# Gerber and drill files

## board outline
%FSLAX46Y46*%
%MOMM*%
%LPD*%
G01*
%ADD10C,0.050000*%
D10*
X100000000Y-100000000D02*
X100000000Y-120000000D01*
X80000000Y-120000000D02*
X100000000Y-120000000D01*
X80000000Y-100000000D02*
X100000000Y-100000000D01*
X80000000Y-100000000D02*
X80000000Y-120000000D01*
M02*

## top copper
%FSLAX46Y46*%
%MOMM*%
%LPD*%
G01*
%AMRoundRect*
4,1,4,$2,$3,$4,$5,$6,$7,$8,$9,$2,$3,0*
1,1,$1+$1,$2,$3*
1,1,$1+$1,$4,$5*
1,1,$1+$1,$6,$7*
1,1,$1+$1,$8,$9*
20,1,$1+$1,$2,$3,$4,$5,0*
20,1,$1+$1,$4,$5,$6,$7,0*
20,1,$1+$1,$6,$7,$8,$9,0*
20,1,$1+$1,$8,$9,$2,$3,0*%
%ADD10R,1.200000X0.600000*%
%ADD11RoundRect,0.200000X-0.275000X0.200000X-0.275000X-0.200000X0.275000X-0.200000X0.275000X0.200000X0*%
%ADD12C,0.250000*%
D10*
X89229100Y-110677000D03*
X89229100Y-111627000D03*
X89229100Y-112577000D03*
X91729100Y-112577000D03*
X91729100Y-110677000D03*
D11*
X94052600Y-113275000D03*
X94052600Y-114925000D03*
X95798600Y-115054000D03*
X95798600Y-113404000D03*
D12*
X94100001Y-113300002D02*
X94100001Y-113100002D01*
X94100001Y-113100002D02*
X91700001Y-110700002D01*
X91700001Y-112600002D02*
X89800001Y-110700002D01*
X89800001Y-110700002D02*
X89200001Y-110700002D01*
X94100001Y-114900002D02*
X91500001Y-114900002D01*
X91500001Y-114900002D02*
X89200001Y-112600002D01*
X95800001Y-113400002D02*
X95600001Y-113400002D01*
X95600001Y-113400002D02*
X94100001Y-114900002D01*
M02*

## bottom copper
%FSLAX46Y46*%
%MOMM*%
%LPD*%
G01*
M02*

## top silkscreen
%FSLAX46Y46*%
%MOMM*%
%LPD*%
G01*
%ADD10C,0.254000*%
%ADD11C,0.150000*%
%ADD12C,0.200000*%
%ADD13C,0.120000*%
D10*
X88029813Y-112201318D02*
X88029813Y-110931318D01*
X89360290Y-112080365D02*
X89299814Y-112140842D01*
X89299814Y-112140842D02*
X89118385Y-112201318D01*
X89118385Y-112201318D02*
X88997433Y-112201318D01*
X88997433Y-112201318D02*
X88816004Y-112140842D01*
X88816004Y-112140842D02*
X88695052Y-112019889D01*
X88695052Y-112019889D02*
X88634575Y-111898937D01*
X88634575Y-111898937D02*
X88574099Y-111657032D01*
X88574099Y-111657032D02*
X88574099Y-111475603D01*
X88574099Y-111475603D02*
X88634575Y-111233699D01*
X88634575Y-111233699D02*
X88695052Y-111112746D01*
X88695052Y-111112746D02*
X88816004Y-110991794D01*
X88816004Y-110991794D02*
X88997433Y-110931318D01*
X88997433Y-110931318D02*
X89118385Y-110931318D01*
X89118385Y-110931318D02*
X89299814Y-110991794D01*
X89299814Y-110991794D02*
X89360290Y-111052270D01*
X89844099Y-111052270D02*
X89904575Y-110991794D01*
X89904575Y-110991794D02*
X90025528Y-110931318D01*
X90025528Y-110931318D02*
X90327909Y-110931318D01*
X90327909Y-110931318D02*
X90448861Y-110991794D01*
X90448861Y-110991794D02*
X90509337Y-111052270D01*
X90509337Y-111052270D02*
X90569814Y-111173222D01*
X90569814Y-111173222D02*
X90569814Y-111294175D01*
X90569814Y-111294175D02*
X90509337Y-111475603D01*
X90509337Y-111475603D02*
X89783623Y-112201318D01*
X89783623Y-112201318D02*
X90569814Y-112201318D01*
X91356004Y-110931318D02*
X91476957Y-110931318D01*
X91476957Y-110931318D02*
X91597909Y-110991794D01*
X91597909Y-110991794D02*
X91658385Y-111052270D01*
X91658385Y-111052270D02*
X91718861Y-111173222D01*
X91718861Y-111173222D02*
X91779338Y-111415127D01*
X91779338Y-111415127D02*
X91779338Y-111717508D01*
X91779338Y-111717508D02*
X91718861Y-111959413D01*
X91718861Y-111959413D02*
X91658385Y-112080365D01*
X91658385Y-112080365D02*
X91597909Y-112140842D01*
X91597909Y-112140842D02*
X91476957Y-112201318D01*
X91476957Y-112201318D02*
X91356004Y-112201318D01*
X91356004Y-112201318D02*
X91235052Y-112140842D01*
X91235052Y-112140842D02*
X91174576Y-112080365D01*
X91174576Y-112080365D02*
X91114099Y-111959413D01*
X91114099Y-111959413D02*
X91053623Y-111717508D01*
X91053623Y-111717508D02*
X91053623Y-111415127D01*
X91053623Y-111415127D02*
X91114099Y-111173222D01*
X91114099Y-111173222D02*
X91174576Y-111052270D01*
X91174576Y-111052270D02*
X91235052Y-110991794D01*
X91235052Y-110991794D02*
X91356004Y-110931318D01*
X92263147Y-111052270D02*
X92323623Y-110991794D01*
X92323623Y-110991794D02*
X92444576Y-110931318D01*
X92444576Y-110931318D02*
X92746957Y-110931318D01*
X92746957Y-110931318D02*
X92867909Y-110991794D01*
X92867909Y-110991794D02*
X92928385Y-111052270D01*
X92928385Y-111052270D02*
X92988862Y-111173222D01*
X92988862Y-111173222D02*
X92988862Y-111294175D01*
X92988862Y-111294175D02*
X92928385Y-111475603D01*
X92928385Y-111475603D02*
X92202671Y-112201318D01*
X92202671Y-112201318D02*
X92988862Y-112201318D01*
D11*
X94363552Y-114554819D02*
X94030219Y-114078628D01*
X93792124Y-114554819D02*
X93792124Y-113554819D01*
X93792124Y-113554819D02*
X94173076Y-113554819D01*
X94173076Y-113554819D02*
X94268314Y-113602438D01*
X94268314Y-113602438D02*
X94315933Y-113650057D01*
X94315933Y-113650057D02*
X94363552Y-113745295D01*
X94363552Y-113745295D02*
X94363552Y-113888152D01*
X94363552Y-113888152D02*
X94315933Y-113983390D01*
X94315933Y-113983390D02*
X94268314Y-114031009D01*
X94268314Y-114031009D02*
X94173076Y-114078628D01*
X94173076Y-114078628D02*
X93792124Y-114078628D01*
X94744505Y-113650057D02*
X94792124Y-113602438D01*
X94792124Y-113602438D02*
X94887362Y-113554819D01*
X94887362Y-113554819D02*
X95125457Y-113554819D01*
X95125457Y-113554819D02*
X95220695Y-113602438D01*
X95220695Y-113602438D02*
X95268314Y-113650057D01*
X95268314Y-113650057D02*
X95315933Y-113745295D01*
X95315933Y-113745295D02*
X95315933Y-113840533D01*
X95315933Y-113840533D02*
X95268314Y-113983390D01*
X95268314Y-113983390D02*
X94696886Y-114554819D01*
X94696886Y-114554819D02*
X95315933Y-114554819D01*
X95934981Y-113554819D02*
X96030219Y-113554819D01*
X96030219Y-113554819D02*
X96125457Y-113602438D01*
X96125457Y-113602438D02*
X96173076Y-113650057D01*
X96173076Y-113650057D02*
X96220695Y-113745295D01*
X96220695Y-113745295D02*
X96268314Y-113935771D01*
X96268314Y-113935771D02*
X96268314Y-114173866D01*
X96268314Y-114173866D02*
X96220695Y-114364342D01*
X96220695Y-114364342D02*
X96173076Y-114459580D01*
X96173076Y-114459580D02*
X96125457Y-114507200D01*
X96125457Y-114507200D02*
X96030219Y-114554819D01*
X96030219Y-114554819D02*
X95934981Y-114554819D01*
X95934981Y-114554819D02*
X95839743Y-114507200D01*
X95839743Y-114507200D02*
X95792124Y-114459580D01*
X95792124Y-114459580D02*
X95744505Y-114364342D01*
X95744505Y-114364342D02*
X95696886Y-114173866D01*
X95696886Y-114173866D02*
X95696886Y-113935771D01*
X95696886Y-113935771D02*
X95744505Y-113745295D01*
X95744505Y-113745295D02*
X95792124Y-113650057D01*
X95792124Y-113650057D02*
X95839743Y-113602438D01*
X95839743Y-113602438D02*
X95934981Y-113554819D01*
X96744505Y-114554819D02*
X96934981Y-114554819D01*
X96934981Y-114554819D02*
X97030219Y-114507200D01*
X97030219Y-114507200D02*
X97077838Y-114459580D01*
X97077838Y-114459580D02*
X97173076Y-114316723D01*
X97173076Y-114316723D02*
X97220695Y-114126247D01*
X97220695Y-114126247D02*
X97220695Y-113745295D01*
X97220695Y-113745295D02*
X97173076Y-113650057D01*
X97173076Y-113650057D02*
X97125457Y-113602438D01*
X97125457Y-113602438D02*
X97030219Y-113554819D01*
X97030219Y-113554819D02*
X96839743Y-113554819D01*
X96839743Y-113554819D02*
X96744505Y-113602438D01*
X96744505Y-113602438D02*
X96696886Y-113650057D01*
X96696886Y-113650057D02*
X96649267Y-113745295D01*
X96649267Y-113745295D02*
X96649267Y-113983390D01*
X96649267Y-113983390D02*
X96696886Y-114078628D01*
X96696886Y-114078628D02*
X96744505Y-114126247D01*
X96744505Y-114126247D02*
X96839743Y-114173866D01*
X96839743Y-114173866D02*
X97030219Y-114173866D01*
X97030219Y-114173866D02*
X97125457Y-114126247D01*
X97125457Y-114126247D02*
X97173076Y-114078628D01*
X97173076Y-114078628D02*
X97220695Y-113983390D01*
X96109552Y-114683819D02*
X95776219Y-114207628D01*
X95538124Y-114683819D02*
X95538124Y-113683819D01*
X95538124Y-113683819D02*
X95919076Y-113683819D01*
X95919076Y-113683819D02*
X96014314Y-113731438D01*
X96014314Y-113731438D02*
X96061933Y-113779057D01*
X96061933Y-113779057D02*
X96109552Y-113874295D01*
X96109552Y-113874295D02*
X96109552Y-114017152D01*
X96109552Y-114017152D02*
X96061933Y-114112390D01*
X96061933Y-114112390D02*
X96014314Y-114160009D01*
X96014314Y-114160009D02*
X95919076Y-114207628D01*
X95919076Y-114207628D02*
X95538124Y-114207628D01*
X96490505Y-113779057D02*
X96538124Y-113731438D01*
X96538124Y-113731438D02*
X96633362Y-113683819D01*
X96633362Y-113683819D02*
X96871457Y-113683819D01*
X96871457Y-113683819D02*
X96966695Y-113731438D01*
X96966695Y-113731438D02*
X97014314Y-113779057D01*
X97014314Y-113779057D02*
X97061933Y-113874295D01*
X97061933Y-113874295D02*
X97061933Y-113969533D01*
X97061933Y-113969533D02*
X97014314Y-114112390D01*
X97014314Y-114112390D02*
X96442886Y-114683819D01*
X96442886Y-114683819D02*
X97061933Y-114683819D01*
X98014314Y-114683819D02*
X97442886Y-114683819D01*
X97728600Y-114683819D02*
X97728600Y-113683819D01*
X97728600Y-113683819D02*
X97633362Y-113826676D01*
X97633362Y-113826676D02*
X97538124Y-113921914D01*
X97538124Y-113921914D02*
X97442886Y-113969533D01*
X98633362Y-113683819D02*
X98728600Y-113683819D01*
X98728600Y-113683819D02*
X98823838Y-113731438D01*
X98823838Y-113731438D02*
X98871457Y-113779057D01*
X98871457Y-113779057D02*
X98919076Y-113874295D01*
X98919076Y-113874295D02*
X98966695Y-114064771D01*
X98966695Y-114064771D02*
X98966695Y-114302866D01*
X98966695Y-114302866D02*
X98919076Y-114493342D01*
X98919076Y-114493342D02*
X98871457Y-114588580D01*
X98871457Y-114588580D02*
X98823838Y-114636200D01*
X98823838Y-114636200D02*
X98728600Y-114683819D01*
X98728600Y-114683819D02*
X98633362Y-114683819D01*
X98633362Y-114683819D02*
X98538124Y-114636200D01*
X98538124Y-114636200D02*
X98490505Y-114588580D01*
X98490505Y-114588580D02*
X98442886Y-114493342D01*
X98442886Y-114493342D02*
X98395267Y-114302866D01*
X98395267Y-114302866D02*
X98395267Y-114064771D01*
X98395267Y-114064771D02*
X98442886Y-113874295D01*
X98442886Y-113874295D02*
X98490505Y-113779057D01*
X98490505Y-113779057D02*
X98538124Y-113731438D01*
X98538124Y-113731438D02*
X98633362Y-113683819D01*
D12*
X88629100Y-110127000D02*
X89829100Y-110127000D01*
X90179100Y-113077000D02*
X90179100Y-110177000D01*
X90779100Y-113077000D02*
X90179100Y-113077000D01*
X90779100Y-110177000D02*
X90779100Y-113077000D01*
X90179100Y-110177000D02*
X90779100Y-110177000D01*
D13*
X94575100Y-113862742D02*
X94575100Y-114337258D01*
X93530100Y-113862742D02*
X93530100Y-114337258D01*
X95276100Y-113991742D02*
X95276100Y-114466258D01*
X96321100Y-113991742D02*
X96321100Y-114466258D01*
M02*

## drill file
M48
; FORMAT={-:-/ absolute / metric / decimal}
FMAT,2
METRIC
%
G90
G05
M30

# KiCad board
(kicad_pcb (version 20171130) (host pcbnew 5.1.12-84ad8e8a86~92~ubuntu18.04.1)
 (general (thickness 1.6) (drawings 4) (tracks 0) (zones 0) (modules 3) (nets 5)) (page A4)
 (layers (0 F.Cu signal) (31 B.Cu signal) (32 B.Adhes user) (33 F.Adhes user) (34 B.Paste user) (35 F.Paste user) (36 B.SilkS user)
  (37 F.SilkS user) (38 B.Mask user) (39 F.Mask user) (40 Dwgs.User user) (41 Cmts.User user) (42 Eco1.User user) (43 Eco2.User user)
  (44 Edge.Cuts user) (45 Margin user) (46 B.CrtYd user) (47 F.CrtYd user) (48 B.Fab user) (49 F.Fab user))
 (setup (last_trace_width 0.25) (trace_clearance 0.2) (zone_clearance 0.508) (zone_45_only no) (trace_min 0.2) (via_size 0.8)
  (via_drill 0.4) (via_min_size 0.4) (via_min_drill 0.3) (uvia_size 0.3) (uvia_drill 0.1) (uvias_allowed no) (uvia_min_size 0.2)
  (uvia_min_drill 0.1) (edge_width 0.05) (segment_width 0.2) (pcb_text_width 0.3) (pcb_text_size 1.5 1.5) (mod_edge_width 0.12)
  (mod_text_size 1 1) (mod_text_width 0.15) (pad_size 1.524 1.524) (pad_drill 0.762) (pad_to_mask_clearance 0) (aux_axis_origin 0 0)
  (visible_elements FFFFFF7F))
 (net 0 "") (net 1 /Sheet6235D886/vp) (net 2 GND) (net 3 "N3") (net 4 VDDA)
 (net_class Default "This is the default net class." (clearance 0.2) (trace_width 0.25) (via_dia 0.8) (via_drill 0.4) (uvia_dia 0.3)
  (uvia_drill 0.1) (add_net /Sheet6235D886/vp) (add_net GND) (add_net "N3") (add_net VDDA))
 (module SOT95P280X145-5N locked (layer F.Cu) (at 90.479100 111.627000)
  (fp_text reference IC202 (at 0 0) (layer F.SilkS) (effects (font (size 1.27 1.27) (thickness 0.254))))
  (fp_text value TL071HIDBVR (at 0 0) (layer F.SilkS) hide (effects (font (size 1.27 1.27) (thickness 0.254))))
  (fp_line (start -1.85 -1.5) (end -0.65 -1.5) (layer F.SilkS) (width 0.2))
  (fp_line (start -0.3 1.45) (end -0.3 -1.45) (layer F.SilkS) (width 0.2))
  (fp_line (start 0.3 1.45) (end -0.3 1.45) (layer F.SilkS) (width 0.2))
  (fp_line (start 0.3 -1.45) (end 0.3 1.45) (layer F.SilkS) (width 0.2))
  (fp_line (start -0.3 -1.45) (end 0.3 -1.45) (layer F.SilkS) (width 0.2))
  (pad 1 smd rect (at -1.25 -0.95 90.000000) (size 0.6 1.2) (layers F.Cu F.Mask F.Paste) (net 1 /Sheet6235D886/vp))
  (pad 2 smd rect (at -1.25 0 90.000000) (size 0.6 1.2) (layers F.Cu F.Mask F.Paste) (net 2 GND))
  (pad 3 smd rect (at -1.25 0.95 90.000000) (size 0.6 1.2) (layers F.Cu F.Mask F.Paste) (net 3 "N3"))
  (pad 4 smd rect (at 1.25 0.95 90.000000) (size 0.6 1.2) (layers F.Cu F.Mask F.Paste) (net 1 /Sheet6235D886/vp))
  (pad 5 smd rect (at 1.25 -0.95 90.000000) (size 0.6 1.2) (layers F.Cu F.Mask F.Paste) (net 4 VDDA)))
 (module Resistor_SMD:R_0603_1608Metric (layer F.Cu) (at 94.052600 114.100000 270.000000)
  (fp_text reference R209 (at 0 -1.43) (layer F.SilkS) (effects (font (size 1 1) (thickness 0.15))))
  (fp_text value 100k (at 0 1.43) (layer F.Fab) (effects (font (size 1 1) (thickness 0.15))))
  (fp_line (start -0.237258 -0.5225) (end 0.237258 -0.5225) (layer F.SilkS) (width 0.12))
  (fp_line (start -0.237258 0.5225) (end 0.237258 0.5225) (layer F.SilkS) (width 0.12))
  (pad 1 smd roundrect (at -0.825 0 270.000000) (size 0.8 0.95) (layers F.Cu F.Mask F.Paste) (roundrect_rratio 0.25) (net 4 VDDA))
  (pad 2 smd roundrect (at 0.825 0 270.000000) (size 0.8 0.95) (layers F.Cu F.Mask F.Paste) (roundrect_rratio 0.25) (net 3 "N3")))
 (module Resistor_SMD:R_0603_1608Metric (layer F.Cu) (at 95.798600 114.229000 270.000000)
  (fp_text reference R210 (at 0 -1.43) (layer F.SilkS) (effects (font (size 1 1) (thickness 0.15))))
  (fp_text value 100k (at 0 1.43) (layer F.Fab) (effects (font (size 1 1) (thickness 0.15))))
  (fp_line (start -0.237258 0.5225) (end 0.237258 0.5225) (layer F.SilkS) (width 0.12))
  (fp_line (start -0.237258 -0.5225) (end 0.237258 -0.5225) (layer F.SilkS) (width 0.12))
  (pad 2 smd roundrect (at 0.825 0 270.000000) (size 0.8 0.95) (layers F.Cu F.Mask F.Paste) (roundrect_rratio 0.25) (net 2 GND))
  (pad 1 smd roundrect (at -0.825 0 270.000000) (size 0.8 0.95) (layers F.Cu F.Mask F.Paste) (roundrect_rratio 0.25) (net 3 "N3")))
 (gr_line (start 100 100) (end 100 120) (layer Edge.Cuts) (width 0.05))
 (gr_line (start 80 120) (end 100 120) (layer Edge.Cuts) (width 0.05))
 (gr_line (start 80 100) (end 100 100) (layer Edge.Cuts) (width 0.05))
 (gr_line (start 80 100) (end 80 120) (layer Edge.Cuts) (width 0.05))
 (segment (start 94.100001 113.300002) (end 94.100001 113.100002) (width 0.250000) (layer F.Cu) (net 4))
 (segment (start 94.100001 113.100002) (end 91.700001 110.700002) (width 0.250000) (layer F.Cu) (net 4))
 (segment (start 91.700001 112.600002) (end 89.800001 110.700002) (width 0.250000) (layer F.Cu) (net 1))
 (segment (start 89.800001 110.700002) (end 89.200001 110.700002) (width 0.250000) (layer F.Cu) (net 1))
 (segment (start 94.100001 114.900002) (end 91.500001 114.900002) (width 0.250000) (layer F.Cu) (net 3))
 (segment (start 91.500001 114.900002) (end 89.200001 112.600002) (width 0.250000) (layer F.Cu) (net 3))
 (segment (start 95.800001 113.400002) (end 95.600001 113.400002) (width 0.250000) (layer F.Cu) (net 3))
 (segment (start 95.600001 113.400002) (end 94.100001 114.900002) (width 0.250000) (layer F.Cu) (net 3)))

